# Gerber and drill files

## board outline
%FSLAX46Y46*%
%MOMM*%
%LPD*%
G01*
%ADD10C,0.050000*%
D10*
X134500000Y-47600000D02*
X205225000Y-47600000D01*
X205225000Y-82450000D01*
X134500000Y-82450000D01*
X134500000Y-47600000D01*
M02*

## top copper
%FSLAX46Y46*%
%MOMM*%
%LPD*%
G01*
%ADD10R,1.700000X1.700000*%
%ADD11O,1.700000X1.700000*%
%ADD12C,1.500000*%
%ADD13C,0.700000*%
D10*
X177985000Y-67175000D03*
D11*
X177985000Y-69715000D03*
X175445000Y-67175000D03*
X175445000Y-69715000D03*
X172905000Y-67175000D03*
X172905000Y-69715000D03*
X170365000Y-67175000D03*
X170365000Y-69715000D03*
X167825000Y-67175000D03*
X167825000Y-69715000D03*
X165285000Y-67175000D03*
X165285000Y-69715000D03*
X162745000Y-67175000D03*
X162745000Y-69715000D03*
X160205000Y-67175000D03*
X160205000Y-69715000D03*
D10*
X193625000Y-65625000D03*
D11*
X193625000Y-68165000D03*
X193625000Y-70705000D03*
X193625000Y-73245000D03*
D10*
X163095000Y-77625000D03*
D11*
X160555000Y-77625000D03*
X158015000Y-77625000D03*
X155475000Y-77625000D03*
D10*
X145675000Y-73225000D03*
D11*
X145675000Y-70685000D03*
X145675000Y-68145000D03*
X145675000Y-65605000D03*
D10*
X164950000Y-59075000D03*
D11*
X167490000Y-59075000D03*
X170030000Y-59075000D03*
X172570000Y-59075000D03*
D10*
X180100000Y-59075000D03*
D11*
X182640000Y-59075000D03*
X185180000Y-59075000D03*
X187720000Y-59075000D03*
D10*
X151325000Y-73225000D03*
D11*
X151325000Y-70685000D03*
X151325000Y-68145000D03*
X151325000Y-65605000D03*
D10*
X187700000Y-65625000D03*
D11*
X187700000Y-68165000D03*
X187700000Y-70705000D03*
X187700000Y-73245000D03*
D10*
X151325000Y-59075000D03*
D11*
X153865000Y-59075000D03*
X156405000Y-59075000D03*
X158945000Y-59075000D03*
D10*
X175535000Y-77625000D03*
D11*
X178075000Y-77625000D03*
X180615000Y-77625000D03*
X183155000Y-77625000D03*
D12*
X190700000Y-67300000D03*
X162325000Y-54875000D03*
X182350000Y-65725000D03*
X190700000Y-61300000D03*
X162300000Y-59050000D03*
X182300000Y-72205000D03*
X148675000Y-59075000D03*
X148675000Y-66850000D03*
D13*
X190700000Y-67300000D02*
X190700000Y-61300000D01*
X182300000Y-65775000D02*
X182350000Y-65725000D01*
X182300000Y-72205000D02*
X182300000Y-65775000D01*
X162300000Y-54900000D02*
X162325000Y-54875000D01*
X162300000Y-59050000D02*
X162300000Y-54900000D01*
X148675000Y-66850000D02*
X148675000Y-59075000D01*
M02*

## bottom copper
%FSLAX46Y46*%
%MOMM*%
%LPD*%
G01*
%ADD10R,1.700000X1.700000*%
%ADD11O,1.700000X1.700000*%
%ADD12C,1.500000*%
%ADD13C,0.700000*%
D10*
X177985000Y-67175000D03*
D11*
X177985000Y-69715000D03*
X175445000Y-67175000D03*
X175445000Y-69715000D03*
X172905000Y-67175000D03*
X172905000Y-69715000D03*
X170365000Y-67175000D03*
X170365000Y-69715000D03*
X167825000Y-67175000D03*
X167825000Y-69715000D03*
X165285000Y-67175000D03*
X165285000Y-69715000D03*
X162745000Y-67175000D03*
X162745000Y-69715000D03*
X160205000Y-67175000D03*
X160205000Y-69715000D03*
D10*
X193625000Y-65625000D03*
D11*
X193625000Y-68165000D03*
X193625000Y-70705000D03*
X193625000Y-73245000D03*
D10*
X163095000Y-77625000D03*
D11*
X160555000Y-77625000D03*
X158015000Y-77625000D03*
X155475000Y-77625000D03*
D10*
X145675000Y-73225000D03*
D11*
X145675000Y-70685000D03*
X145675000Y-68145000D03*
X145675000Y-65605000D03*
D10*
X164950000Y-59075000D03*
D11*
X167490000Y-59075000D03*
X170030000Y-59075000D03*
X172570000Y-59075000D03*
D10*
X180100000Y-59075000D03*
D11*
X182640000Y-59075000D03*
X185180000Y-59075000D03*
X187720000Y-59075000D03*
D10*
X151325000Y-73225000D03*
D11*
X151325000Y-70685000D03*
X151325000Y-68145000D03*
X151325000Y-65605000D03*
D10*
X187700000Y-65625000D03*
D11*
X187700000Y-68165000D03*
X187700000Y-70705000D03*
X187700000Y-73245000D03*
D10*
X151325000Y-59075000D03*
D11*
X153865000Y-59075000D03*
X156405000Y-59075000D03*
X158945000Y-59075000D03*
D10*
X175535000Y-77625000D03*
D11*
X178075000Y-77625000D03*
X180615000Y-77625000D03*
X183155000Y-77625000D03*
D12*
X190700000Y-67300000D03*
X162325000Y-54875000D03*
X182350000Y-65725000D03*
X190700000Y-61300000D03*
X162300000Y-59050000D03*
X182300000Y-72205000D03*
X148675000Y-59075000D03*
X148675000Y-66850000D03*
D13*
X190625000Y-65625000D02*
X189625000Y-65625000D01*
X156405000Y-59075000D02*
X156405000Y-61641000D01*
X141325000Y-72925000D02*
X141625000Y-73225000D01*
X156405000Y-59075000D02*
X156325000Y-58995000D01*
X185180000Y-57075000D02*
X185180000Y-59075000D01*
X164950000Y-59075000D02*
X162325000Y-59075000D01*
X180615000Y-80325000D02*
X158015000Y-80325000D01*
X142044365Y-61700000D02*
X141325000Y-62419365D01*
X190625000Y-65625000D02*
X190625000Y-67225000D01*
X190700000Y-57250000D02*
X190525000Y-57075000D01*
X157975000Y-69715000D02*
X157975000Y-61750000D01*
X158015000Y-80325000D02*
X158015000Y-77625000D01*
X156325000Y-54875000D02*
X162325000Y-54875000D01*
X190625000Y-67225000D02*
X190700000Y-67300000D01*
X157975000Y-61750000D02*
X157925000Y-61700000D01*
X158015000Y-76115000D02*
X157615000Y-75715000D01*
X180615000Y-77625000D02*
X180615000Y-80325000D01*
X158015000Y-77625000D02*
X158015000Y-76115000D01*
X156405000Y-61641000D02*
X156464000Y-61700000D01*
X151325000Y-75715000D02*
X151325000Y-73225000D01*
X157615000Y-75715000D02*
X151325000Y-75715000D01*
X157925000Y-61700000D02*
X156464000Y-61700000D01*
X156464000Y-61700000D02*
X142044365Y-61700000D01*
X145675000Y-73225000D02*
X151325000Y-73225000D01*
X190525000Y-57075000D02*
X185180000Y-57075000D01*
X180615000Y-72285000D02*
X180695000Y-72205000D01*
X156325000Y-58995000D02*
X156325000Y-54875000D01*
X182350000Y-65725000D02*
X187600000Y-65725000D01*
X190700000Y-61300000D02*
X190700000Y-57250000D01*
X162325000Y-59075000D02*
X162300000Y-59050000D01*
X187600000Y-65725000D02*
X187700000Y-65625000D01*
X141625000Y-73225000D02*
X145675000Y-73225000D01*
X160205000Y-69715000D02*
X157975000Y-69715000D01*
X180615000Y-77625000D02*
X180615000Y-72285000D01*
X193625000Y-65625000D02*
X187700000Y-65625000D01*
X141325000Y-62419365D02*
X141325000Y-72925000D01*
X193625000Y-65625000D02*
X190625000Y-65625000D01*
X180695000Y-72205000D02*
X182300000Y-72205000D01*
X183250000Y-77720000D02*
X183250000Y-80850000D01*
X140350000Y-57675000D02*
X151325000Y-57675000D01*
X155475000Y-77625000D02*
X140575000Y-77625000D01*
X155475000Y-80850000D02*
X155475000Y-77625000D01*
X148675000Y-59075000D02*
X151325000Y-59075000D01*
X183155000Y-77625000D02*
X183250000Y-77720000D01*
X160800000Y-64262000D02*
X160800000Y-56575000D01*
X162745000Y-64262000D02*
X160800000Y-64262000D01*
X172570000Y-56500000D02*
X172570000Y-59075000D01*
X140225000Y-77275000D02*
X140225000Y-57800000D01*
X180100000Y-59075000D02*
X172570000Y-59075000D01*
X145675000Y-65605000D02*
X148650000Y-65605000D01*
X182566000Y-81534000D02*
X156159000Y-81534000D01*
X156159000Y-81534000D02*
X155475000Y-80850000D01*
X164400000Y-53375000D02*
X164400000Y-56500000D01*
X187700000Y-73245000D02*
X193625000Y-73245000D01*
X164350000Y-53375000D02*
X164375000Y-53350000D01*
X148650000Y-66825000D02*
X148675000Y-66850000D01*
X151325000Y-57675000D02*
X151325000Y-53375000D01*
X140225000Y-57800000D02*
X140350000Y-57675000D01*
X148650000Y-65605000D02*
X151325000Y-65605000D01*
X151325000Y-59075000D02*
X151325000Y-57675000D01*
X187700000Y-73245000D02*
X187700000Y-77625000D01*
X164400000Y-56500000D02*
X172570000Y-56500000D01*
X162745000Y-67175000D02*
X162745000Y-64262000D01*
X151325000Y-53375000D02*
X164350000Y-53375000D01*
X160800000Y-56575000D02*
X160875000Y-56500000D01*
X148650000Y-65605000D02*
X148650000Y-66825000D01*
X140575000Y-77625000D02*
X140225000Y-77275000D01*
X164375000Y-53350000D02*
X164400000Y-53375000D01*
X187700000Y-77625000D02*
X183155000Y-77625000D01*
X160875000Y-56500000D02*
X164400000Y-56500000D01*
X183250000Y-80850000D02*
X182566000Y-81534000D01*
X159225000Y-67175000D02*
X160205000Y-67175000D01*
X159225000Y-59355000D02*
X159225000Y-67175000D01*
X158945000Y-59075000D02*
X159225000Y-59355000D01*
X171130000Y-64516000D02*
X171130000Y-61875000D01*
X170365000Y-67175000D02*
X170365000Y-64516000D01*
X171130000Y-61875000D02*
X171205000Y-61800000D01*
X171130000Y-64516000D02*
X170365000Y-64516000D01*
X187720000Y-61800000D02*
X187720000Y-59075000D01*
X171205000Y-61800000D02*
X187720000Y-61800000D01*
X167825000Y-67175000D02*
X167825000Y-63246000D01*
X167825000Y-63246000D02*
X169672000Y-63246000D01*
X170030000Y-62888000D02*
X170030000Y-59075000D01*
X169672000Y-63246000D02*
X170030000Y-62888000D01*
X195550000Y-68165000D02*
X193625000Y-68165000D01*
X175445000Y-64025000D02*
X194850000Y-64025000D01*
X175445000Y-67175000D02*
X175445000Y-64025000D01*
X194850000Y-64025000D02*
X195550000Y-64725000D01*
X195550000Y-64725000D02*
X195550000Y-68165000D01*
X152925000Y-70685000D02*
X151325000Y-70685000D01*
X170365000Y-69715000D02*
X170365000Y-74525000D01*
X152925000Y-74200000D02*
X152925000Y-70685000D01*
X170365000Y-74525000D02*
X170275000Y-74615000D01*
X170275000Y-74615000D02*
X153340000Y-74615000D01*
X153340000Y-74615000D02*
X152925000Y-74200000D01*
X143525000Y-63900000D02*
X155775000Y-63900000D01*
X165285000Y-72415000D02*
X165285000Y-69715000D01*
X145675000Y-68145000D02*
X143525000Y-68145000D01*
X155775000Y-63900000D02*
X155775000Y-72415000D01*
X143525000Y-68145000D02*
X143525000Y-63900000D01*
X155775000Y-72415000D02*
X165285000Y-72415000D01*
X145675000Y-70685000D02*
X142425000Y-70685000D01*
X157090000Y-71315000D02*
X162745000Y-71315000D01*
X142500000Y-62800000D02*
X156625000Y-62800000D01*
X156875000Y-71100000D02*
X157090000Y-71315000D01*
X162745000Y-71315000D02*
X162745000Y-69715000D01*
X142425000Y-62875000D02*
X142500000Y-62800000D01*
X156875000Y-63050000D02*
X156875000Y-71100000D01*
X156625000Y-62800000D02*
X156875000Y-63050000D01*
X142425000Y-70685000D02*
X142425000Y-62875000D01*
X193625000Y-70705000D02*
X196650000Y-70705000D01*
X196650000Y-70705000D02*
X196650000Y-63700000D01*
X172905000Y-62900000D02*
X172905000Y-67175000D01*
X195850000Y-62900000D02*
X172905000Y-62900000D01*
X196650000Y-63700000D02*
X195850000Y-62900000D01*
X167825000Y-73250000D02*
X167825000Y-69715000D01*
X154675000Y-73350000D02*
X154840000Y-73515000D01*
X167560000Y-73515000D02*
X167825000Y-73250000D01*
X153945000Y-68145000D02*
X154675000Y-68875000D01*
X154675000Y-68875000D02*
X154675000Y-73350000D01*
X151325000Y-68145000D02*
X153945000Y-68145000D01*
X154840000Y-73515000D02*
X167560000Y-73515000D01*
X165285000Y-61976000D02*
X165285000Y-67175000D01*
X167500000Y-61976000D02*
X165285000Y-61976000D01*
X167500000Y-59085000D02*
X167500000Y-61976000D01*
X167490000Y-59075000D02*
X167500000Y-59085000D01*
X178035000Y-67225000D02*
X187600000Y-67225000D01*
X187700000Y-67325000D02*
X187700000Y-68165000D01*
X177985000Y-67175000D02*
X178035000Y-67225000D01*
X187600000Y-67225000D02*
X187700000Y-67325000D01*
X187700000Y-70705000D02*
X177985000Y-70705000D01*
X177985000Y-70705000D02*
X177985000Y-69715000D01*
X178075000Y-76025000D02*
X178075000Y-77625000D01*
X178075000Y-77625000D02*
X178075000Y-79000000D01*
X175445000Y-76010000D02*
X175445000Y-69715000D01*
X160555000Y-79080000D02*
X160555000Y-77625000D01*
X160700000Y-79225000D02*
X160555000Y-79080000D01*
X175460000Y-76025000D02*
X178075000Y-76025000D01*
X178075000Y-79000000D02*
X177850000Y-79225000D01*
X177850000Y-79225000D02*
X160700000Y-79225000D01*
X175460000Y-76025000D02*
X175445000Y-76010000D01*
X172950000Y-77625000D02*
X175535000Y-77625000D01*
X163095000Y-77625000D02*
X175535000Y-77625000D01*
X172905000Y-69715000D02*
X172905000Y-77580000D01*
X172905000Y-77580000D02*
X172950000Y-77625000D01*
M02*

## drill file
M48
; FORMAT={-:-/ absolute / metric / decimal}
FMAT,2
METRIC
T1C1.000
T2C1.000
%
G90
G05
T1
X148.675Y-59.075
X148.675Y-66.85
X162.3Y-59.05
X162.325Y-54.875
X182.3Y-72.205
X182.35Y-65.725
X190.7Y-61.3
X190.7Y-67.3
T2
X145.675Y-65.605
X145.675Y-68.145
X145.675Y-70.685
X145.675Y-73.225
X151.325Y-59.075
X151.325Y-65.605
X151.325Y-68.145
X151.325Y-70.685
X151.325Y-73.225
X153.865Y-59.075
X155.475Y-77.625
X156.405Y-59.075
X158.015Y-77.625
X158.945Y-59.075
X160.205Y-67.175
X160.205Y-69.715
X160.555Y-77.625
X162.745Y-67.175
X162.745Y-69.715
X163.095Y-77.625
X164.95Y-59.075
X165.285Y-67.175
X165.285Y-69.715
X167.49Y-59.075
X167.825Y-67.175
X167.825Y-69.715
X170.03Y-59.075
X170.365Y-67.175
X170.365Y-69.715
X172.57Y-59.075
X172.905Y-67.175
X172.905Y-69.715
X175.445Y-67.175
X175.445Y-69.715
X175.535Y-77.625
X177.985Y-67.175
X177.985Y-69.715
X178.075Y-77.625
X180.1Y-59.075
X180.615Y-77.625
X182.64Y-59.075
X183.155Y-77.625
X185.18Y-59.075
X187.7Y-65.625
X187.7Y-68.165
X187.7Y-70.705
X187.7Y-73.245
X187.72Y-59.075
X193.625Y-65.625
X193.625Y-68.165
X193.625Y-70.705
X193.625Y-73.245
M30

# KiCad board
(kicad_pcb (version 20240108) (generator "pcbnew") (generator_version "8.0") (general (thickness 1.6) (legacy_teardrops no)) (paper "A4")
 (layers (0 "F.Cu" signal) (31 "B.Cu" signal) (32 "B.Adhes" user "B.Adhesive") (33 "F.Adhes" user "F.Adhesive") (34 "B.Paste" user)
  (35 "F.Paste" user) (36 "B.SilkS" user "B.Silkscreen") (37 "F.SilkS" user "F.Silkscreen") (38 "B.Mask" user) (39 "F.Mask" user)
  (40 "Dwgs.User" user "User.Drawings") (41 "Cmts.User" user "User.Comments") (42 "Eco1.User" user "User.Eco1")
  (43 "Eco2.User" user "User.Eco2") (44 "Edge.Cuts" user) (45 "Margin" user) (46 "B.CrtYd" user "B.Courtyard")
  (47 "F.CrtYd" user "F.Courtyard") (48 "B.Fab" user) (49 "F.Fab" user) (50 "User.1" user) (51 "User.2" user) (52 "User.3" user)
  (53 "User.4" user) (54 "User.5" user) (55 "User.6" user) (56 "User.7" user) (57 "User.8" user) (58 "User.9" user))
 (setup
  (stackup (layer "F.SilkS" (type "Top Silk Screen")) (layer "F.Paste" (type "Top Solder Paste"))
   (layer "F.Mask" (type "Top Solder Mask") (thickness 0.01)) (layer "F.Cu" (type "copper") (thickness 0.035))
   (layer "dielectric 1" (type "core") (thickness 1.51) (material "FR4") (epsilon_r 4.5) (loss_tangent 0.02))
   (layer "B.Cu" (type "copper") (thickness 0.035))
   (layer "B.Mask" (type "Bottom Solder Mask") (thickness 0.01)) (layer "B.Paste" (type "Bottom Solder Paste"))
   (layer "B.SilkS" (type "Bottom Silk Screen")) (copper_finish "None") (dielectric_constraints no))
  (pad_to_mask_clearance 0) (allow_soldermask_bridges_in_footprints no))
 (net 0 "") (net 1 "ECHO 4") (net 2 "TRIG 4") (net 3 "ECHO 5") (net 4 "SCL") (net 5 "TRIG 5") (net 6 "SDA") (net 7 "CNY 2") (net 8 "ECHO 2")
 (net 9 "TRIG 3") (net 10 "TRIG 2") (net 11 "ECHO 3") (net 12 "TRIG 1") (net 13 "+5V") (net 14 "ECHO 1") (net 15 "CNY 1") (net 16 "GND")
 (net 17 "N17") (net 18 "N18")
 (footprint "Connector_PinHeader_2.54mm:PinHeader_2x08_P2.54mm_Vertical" (layer "F.Cu") (at 177.985 67.175 -90)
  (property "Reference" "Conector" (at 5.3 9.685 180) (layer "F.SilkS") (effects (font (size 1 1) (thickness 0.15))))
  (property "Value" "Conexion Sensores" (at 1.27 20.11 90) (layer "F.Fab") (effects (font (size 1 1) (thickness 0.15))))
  (pad "1" thru_hole rect (at 0 0 270) (size 1.7 1.7) (drill 1) (layers "*.Cu" "*.Mask") (remove_unused_layers no) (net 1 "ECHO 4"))
  (pad "2" thru_hole oval (at 2.54 0 270) (size 1.7 1.7) (drill 1) (layers "*.Cu" "*.Mask") (remove_unused_layers no) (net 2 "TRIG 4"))
  (pad "3" thru_hole oval (at 0 2.54 270) (size 1.7 1.7) (drill 1) (layers "*.Cu" "*.Mask") (remove_unused_layers no) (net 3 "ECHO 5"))
  (pad "4" thru_hole oval (at 2.54 2.54 270) (size 1.7 1.7) (drill 1) (layers "*.Cu" "*.Mask") (remove_unused_layers no) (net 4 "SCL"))
  (pad "5" thru_hole oval (at 0 5.08 270) (size 1.7 1.7) (drill 1) (layers "*.Cu" "*.Mask") (remove_unused_layers no) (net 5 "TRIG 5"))
  (pad "6" thru_hole oval (at 2.54 5.08 270) (size 1.7 1.7) (drill 1) (layers "*.Cu" "*.Mask") (remove_unused_layers no) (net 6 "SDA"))
  (pad "7" thru_hole oval (at 0 7.62 270) (size 1.7 1.7) (drill 1) (layers "*.Cu" "*.Mask") (remove_unused_layers no) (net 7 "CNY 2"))
  (pad "8" thru_hole oval (at 2.54 7.62 270) (size 1.7 1.7) (drill 1) (layers "*.Cu" "*.Mask") (remove_unused_layers no) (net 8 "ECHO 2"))
  (pad "9" thru_hole oval (at 0 10.16 270) (size 1.7 1.7) (drill 1) (layers "*.Cu" "*.Mask") (remove_unused_layers no) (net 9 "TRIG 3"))
  (pad "10" thru_hole oval (at 2.54 10.16 270) (size 1.7 1.7) (drill 1) (layers "*.Cu" "*.Mask") (remove_unused_layers no) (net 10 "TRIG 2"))
  (pad "11" thru_hole oval (at 0 12.7 270) (size 1.7 1.7) (drill 1) (layers "*.Cu" "*.Mask") (remove_unused_layers no) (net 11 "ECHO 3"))
  (pad "12" thru_hole oval (at 2.54 12.7 270) (size 1.7 1.7) (drill 1) (layers "*.Cu" "*.Mask") (remove_unused_layers no) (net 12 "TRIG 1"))
  (pad "13" thru_hole oval (at 0 15.24 270) (size 1.7 1.7) (drill 1) (layers "*.Cu" "*.Mask") (remove_unused_layers no) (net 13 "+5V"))
  (pad "14" thru_hole oval (at 2.54 15.24 270) (size 1.7 1.7) (drill 1) (layers "*.Cu" "*.Mask") (remove_unused_layers no) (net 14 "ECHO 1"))
  (pad "15" thru_hole oval (at 0 17.78 270) (size 1.7 1.7) (drill 1) (layers "*.Cu" "*.Mask") (remove_unused_layers no) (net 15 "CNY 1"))
  (pad "16" thru_hole oval (at 2.54 17.78 270) (size 1.7 1.7) (drill 1) (layers "*.Cu" "*.Mask") (remove_unused_layers no) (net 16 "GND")))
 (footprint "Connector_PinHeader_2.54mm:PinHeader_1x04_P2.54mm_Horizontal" (layer "F.Cu") (at 193.625 65.625)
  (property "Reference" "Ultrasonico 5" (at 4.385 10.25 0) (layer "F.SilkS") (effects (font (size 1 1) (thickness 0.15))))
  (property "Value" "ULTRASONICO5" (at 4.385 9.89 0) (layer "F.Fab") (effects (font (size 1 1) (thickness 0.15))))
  (pad "1" thru_hole rect (at 0 0) (size 1.7 1.7) (drill 1) (layers "*.Cu" "*.Mask") (remove_unused_layers no) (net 16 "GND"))
  (pad "2" thru_hole oval (at 0 2.54) (size 1.7 1.7) (drill 1) (layers "*.Cu" "*.Mask") (remove_unused_layers no) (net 3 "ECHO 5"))
  (pad "3" thru_hole oval (at 0 5.08) (size 1.7 1.7) (drill 1) (layers "*.Cu" "*.Mask") (remove_unused_layers no) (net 5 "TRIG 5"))
  (pad "4" thru_hole oval (at 0 7.62) (size 1.7 1.7) (drill 1) (layers "*.Cu" "*.Mask") (remove_unused_layers no) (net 13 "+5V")))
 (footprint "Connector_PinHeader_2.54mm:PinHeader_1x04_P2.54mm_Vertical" (layer "F.Cu") (at 163.095 77.625 -90)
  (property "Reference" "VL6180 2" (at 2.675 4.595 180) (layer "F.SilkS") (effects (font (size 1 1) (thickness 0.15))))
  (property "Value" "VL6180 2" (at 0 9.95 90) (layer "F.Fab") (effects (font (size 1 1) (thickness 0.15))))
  (pad "1" thru_hole rect (at 0 0 270) (size 1.7 1.7) (drill 1) (layers "*.Cu" "*.Mask") (remove_unused_layers no) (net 6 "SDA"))
  (pad "2" thru_hole oval (at 0 2.54 270) (size 1.7 1.7) (drill 1) (layers "*.Cu" "*.Mask") (remove_unused_layers no) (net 4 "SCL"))
  (pad "3" thru_hole oval (at 0 5.08 270) (size 1.7 1.7) (drill 1) (layers "*.Cu" "*.Mask") (remove_unused_layers no) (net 16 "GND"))
  (pad "4" thru_hole oval (at 0 7.62 270) (size 1.7 1.7) (drill 1) (layers "*.Cu" "*.Mask") (remove_unused_layers no) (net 13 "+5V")))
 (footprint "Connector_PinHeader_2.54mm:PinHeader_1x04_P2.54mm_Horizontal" (layer "F.Cu") (at 145.675 73.225 180)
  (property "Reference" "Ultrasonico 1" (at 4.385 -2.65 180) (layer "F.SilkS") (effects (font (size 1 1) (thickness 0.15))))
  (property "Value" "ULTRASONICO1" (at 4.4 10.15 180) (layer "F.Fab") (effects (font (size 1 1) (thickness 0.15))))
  (pad "1" thru_hole rect (at 0 0 180) (size 1.7 1.7) (drill 1) (layers "*.Cu" "*.Mask") (remove_unused_layers no) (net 16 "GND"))
  (pad "2" thru_hole oval (at 0 2.54 180) (size 1.7 1.7) (drill 1) (layers "*.Cu" "*.Mask") (remove_unused_layers no) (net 14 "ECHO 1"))
  (pad "3" thru_hole oval (at 0 5.08 180) (size 1.7 1.7) (drill 1) (layers "*.Cu" "*.Mask") (remove_unused_layers no) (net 12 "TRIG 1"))
  (pad "4" thru_hole oval (at 0 7.62 180) (size 1.7 1.7) (drill 1) (layers "*.Cu" "*.Mask") (remove_unused_layers no) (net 13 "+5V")))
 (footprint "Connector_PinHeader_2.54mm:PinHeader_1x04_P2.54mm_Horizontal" (layer "F.Cu") (at 164.95 59.075 90)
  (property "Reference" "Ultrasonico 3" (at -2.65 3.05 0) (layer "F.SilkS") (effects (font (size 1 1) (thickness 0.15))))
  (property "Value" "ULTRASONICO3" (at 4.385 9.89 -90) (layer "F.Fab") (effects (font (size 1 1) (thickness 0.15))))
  (pad "1" thru_hole rect (at 0 0 90) (size 1.7 1.7) (drill 1) (layers "*.Cu" "*.Mask") (remove_unused_layers no) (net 16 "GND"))
  (pad "2" thru_hole oval (at 0 2.54 90) (size 1.7 1.7) (drill 1) (layers "*.Cu" "*.Mask") (remove_unused_layers no) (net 11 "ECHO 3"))
  (pad "3" thru_hole oval (at 0 5.08 90) (size 1.7 1.7) (drill 1) (layers "*.Cu" "*.Mask") (remove_unused_layers no) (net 9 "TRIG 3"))
  (pad "4" thru_hole oval (at 0 7.62 90) (size 1.7 1.7) (drill 1) (layers "*.Cu" "*.Mask") (remove_unused_layers no) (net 13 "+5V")))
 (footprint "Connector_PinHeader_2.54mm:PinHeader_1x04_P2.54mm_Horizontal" (layer "F.Cu") (at 180.1 59.075 90)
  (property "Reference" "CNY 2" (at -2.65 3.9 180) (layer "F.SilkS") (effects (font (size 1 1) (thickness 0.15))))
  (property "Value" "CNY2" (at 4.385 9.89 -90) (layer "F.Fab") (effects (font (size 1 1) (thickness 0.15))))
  (pad "1" thru_hole rect (at 0 0 90) (size 1.7 1.7) (drill 1) (layers "*.Cu" "*.Mask") (remove_unused_layers no) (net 13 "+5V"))
  (pad "2" thru_hole oval (at 0 2.54 90) (size 1.7 1.7) (drill 1) (layers "*.Cu" "*.Mask") (remove_unused_layers no) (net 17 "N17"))
  (pad "3" thru_hole oval (at 0 5.08 90) (size 1.7 1.7) (drill 1) (layers "*.Cu" "*.Mask") (remove_unused_layers no) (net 16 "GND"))
  (pad "4" thru_hole oval (at 0 7.62 90) (size 1.7 1.7) (drill 1) (layers "*.Cu" "*.Mask") (remove_unused_layers no) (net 7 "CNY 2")))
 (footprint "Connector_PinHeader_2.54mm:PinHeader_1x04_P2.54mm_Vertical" (layer "F.Cu") (at 151.325 73.225 180)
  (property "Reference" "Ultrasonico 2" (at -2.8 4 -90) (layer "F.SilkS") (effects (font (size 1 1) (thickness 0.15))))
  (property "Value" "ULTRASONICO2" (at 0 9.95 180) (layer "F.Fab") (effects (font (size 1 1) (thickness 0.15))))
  (pad "1" thru_hole rect (at 0 0 180) (size 1.7 1.7) (drill 1) (layers "*.Cu" "*.Mask") (remove_unused_layers no) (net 16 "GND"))
  (pad "2" thru_hole oval (at 0 2.54 180) (size 1.7 1.7) (drill 1) (layers "*.Cu" "*.Mask") (remove_unused_layers no) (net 8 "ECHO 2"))
  (pad "3" thru_hole oval (at 0 5.08 180) (size 1.7 1.7) (drill 1) (layers "*.Cu" "*.Mask") (remove_unused_layers no) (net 10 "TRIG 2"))
  (pad "4" thru_hole oval (at 0 7.62 180) (size 1.7 1.7) (drill 1) (layers "*.Cu" "*.Mask") (remove_unused_layers no) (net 13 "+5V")))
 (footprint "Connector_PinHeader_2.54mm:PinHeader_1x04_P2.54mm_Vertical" (layer "F.Cu") (at 187.7 65.625)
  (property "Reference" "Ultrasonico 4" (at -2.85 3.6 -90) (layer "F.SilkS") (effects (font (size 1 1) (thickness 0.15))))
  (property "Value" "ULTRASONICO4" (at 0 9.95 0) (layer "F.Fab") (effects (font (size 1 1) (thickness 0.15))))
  (pad "1" thru_hole rect (at 0 0) (size 1.7 1.7) (drill 1) (layers "*.Cu" "*.Mask") (remove_unused_layers no) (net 16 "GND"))
  (pad "2" thru_hole oval (at 0 2.54) (size 1.7 1.7) (drill 1) (layers "*.Cu" "*.Mask") (remove_unused_layers no) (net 1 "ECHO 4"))
  (pad "3" thru_hole oval (at 0 5.08) (size 1.7 1.7) (drill 1) (layers "*.Cu" "*.Mask") (remove_unused_layers no) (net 2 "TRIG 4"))
  (pad "4" thru_hole oval (at 0 7.62) (size 1.7 1.7) (drill 1) (layers "*.Cu" "*.Mask") (remove_unused_layers no) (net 13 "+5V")))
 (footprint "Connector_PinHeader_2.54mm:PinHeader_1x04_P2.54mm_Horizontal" (layer "F.Cu") (at 151.325 59.075 90)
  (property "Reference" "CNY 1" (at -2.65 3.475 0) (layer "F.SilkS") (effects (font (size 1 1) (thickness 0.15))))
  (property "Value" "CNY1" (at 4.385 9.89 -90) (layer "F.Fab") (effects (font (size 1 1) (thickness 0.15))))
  (pad "1" thru_hole rect (at 0 0 90) (size 1.7 1.7) (drill 1) (layers "*.Cu" "*.Mask") (remove_unused_layers no) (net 13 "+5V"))
  (pad "2" thru_hole oval (at 0 2.54 90) (size 1.7 1.7) (drill 1) (layers "*.Cu" "*.Mask") (remove_unused_layers no) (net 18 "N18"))
  (pad "3" thru_hole oval (at 0 5.08 90) (size 1.7 1.7) (drill 1) (layers "*.Cu" "*.Mask") (remove_unused_layers no) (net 16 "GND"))
  (pad "4" thru_hole oval (at 0 7.62 90) (size 1.7 1.7) (drill 1) (layers "*.Cu" "*.Mask") (remove_unused_layers no) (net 15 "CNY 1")))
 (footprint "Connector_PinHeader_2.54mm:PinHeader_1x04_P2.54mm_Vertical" (layer "F.Cu") (at 175.535 77.625 90)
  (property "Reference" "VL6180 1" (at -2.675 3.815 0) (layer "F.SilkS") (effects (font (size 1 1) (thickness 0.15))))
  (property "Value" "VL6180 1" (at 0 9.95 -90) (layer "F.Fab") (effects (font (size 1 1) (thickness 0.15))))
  (pad "1" thru_hole rect (at 0 0 90) (size 1.7 1.7) (drill 1) (layers "*.Cu" "*.Mask") (remove_unused_layers no) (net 6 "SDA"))
  (pad "2" thru_hole oval (at 0 2.54 90) (size 1.7 1.7) (drill 1) (layers "*.Cu" "*.Mask") (remove_unused_layers no) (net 4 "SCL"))
  (pad "3" thru_hole oval (at 0 5.08 90) (size 1.7 1.7) (drill 1) (layers "*.Cu" "*.Mask") (remove_unused_layers no) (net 16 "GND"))
  (pad "4" thru_hole oval (at 0 7.62 90) (size 1.7 1.7) (drill 1) (layers "*.Cu" "*.Mask") (remove_unused_layers no) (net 13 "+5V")))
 (gr_rect (start 134.5 47.6) (end 205.225 82.45) (stroke (width 0.05) (type default)) (fill none) (layer "Edge.Cuts"))
 (segment (start 190.7 67.3) (end 190.7 61.3) (width 0.7) (layer "F.Cu") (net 16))
 (segment (start 182.3 65.775) (end 182.35 65.725) (width 0.7) (layer "F.Cu") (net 16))
 (segment (start 182.3 72.205) (end 182.3 65.775) (width 0.7) (layer "F.Cu") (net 16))
 (segment (start 162.3 54.9) (end 162.325 54.875) (width 0.7) (layer "F.Cu") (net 16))
 (segment (start 162.3 59.05) (end 162.3 54.9) (width 0.7) (layer "F.Cu") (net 16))
 (via (at 190.7 67.3) (size 1.5) (drill 1) (layers "F.Cu" "B.Cu") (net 16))
 (via (at 162.325 54.875) (size 1.5) (drill 1) (layers "F.Cu" "B.Cu") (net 16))
 (via (at 182.35 65.725) (size 1.5) (drill 1) (layers "F.Cu" "B.Cu") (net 16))
 (via (at 190.7 61.3) (size 1.5) (drill 1) (layers "F.Cu" "B.Cu") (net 16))
 (via (at 162.3 59.05) (size 1.5) (drill 1) (layers "F.Cu" "B.Cu") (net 16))
 (via (at 182.3 72.205) (size 1.5) (drill 1) (layers "F.Cu" "B.Cu") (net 16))
 (segment (start 190.625 65.625) (end 189.625 65.625) (width 0.7) (layer "B.Cu") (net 16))
 (segment (start 156.405 59.075) (end 156.405 61.641) (width 0.7) (layer "B.Cu") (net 16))
 (segment (start 141.325 72.925) (end 141.625 73.225) (width 0.7) (layer "B.Cu") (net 16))
 (segment (start 156.405 59.075) (end 156.325 58.995) (width 0.7) (layer "B.Cu") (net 16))
 (segment (start 185.18 57.075) (end 185.18 59.075) (width 0.7) (layer "B.Cu") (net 16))
 (segment (start 164.95 59.075) (end 162.325 59.075) (width 0.7) (layer "B.Cu") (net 16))
 (segment (start 180.615 80.325) (end 158.015 80.325) (width 0.7) (layer "B.Cu") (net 16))
 (segment (start 142.044365 61.7) (end 141.325 62.419365) (width 0.7) (layer "B.Cu") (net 16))
 (segment (start 190.625 65.625) (end 190.625 67.225) (width 0.7) (layer "B.Cu") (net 16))
 (segment (start 190.7 57.25) (end 190.525 57.075) (width 0.7) (layer "B.Cu") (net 16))
 (segment (start 157.975 69.715) (end 157.975 61.75) (width 0.7) (layer "B.Cu") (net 16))
 (segment (start 158.015 80.325) (end 158.015 77.625) (width 0.7) (layer "B.Cu") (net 16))
 (segment (start 156.325 54.875) (end 162.325 54.875) (width 0.7) (layer "B.Cu") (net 16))
 (segment (start 190.625 67.225) (end 190.7 67.3) (width 0.7) (layer "B.Cu") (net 16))
 (segment (start 157.975 61.75) (end 157.925 61.7) (width 0.7) (layer "B.Cu") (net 16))
 (segment (start 158.015 76.115) (end 157.615 75.715) (width 0.7) (layer "B.Cu") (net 16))
 (segment (start 180.615 77.625) (end 180.615 80.325) (width 0.7) (layer "B.Cu") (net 16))
 (segment (start 158.015 77.625) (end 158.015 76.115) (width 0.7) (layer "B.Cu") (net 16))
 (segment (start 156.405 61.641) (end 156.464 61.7) (width 0.7) (layer "B.Cu") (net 16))
 (segment (start 151.325 75.715) (end 151.325 73.225) (width 0.7) (layer "B.Cu") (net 16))
 (segment (start 157.615 75.715) (end 151.325 75.715) (width 0.7) (layer "B.Cu") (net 16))
 (segment (start 157.925 61.7) (end 156.464 61.7) (width 0.7) (layer "B.Cu") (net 16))
 (segment (start 156.464 61.7) (end 142.044365 61.7) (width 0.7) (layer "B.Cu") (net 16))
 (segment (start 145.675 73.225) (end 151.325 73.225) (width 0.7) (layer "B.Cu") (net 16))
 (segment (start 190.525 57.075) (end 185.18 57.075) (width 0.7) (layer "B.Cu") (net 16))
 (segment (start 180.615 72.285) (end 180.695 72.205) (width 0.7) (layer "B.Cu") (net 16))
 (segment (start 156.325 58.995) (end 156.325 54.875) (width 0.7) (layer "B.Cu") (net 16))
 (segment (start 182.35 65.725) (end 187.6 65.725) (width 0.7) (layer "B.Cu") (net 16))
 (segment (start 190.7 61.3) (end 190.7 57.25) (width 0.7) (layer "B.Cu") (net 16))
 (segment (start 162.325 59.075) (end 162.3 59.05) (width 0.7) (layer "B.Cu") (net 16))
 (segment (start 187.6 65.725) (end 187.7 65.625) (width 0.7) (layer "B.Cu") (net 16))
 (segment (start 141.625 73.225) (end 145.675 73.225) (width 0.7) (layer "B.Cu") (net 16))
 (segment (start 160.205 69.715) (end 157.975 69.715) (width 0.7) (layer "B.Cu") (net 16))
 (segment (start 180.615 77.625) (end 180.615 72.285) (width 0.7) (layer "B.Cu") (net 16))
 (segment (start 193.625 65.625) (end 187.7 65.625) (width 0.7) (layer "B.Cu") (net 16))
 (segment (start 141.325 62.419365) (end 141.325 72.925) (width 0.7) (layer "B.Cu") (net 16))
 (segment (start 193.625 65.625) (end 190.625 65.625) (width 0.7) (layer "B.Cu") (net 16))
 (segment (start 180.695 72.205) (end 182.3 72.205) (width 0.7) (layer "B.Cu") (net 16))
 (segment (start 148.675 66.85) (end 148.675 59.075) (width 0.7) (layer "F.Cu") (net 13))
 (via (at 148.675 59.075) (size 1.5) (drill 1) (layers "F.Cu" "B.Cu") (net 13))
 (via (at 148.675 66.85) (size 1.5) (drill 1) (layers "F.Cu" "B.Cu") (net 13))
 (segment (start 183.25 77.72) (end 183.25 80.85) (width 0.7) (layer "B.Cu") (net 13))
 (segment (start 140.35 57.675) (end 151.325 57.675) (width 0.7) (layer "B.Cu") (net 13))
 (segment (start 155.475 77.625) (end 140.575 77.625) (width 0.7) (layer "B.Cu") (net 13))
 (segment (start 155.475 80.85) (end 155.475 77.625) (width 0.7) (layer "B.Cu") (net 13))
 (segment (start 148.675 59.075) (end 151.325 59.075) (width 0.7) (layer "B.Cu") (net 13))
 (segment (start 183.155 77.625) (end 183.25 77.72) (width 0.7) (layer "B.Cu") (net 13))
 (segment (start 160.8 64.262) (end 160.8 56.575) (width 0.7) (layer "B.Cu") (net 13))
 (segment (start 162.745 64.262) (end 160.8 64.262) (width 0.7) (layer "B.Cu") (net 13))
 (segment (start 172.57 56.5) (end 172.57 59.075) (width 0.7) (layer "B.Cu") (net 13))
 (segment (start 140.225 77.275) (end 140.225 57.8) (width 0.7) (layer "B.Cu") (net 13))
 (segment (start 180.1 59.075) (end 172.57 59.075) (width 0.7) (layer "B.Cu") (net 13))
 (segment (start 145.675 65.605) (end 148.65 65.605) (width 0.7) (layer "B.Cu") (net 13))
 (segment (start 182.566 81.534) (end 156.159 81.534) (width 0.7) (layer "B.Cu") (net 13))
 (segment (start 156.159 81.534) (end 155.475 80.85) (width 0.7) (layer "B.Cu") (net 13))
 (segment (start 164.4 53.375) (end 164.4 56.5) (width 0.7) (layer "B.Cu") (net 13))
 (segment (start 187.7 73.245) (end 193.625 73.245) (width 0.7) (layer "B.Cu") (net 13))
 (segment (start 164.35 53.375) (end 164.375 53.35) (width 0.7) (layer "B.Cu") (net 13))
 (segment (start 148.65 66.825) (end 148.675 66.85) (width 0.7) (layer "B.Cu") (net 13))
 (segment (start 151.325 57.675) (end 151.325 53.375) (width 0.7) (layer "B.Cu") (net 13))
 (segment (start 140.225 57.8) (end 140.35 57.675) (width 0.7) (layer "B.Cu") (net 13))
 (segment (start 148.65 65.605) (end 151.325 65.605) (width 0.7) (layer "B.Cu") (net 13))
 (segment (start 151.325 59.075) (end 151.325 57.675) (width 0.7) (layer "B.Cu") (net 13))
 (segment (start 187.7 73.245) (end 187.7 77.625) (width 0.7) (layer "B.Cu") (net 13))
 (segment (start 164.4 56.5) (end 172.57 56.5) (width 0.7) (layer "B.Cu") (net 13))
 (segment (start 162.745 67.175) (end 162.745 64.262) (width 0.7) (layer "B.Cu") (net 13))
 (segment (start 151.325 53.375) (end 164.35 53.375) (width 0.7) (layer "B.Cu") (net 13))
 (segment (start 160.8 56.575) (end 160.875 56.5) (width 0.7) (layer "B.Cu") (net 13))
 (segment (start 148.65 65.605) (end 148.65 66.825) (width 0.7) (layer "B.Cu") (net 13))
 (segment (start 140.575 77.625) (end 140.225 77.275) (width 0.7) (layer "B.Cu") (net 13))
 (segment (start 164.375 53.35) (end 164.4 53.375) (width 0.7) (layer "B.Cu") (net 13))
 (segment (start 187.7 77.625) (end 183.155 77.625) (width 0.7) (layer "B.Cu") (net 13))
 (segment (start 160.875 56.5) (end 164.4 56.5) (width 0.7) (layer "B.Cu") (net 13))
 (segment (start 183.25 80.85) (end 182.566 81.534) (width 0.7) (layer "B.Cu") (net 13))
 (segment (start 159.225 67.175) (end 160.205 67.175) (width 0.7) (layer "B.Cu") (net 15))
 (segment (start 159.225 59.355) (end 159.225 67.175) (width 0.7) (layer "B.Cu") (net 15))
 (segment (start 158.945 59.075) (end 159.225 59.355) (width 0.7) (layer "B.Cu") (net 15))
 (segment (start 171.13 64.516) (end 171.13 61.875) (width 0.7) (layer "B.Cu") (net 7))
 (segment (start 170.365 67.175) (end 170.365 64.516) (width 0.7) (layer "B.Cu") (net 7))
 (segment (start 171.13 61.875) (end 171.205 61.8) (width 0.7) (layer "B.Cu") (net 7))
 (segment (start 171.13 64.516) (end 170.365 64.516) (width 0.7) (layer "B.Cu") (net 7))
 (segment (start 187.72 61.8) (end 187.72 59.075) (width 0.7) (layer "B.Cu") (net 7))
 (segment (start 171.205 61.8) (end 187.72 61.8) (width 0.7) (layer "B.Cu") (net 7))
 (segment (start 167.825 67.175) (end 167.825 63.246) (width 0.7) (layer "B.Cu") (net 9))
 (segment (start 167.825 63.246) (end 169.672 63.246) (width 0.7) (layer "B.Cu") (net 9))
 (segment (start 170.03 62.888) (end 170.03 59.075) (width 0.7) (layer "B.Cu") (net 9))
 (segment (start 169.672 63.246) (end 170.03 62.888) (width 0.7) (layer "B.Cu") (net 9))
 (segment (start 195.55 68.165) (end 193.625 68.165) (width 0.7) (layer "B.Cu") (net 3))
 (segment (start 175.445 64.025) (end 194.85 64.025) (width 0.7) (layer "B.Cu") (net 3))
 (segment (start 175.445 67.175) (end 175.445 64.025) (width 0.7) (layer "B.Cu") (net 3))
 (segment (start 194.85 64.025) (end 195.55 64.725) (width 0.7) (layer "B.Cu") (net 3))
 (segment (start 195.55 64.725) (end 195.55 68.165) (width 0.7) (layer "B.Cu") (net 3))
 (segment (start 152.925 70.685) (end 151.325 70.685) (width 0.7) (layer "B.Cu") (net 8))
 (segment (start 170.365 69.715) (end 170.365 74.525) (width 0.7) (layer "B.Cu") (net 8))
 (segment (start 152.925 74.2) (end 152.925 70.685) (width 0.7) (layer "B.Cu") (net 8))
 (segment (start 170.365 74.525) (end 170.275 74.615) (width 0.7) (layer "B.Cu") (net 8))
 (segment (start 170.275 74.615) (end 153.34 74.615) (width 0.7) (layer "B.Cu") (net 8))
 (segment (start 153.34 74.615) (end 152.925 74.2) (width 0.7) (layer "B.Cu") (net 8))
 (segment (start 143.525 63.9) (end 155.775 63.9) (width 0.7) (layer "B.Cu") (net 12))
 (segment (start 165.285 72.415) (end 165.285 69.715) (width 0.7) (layer "B.Cu") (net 12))
 (segment (start 145.675 68.145) (end 143.525 68.145) (width 0.7) (layer "B.Cu") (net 12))
 (segment (start 155.775 63.9) (end 155.775 72.415) (width 0.7) (layer "B.Cu") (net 12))
 (segment (start 143.525 68.145) (end 143.525 63.9) (width 0.7) (layer "B.Cu") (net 12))
 (segment (start 155.775 72.415) (end 165.285 72.415) (width 0.7) (layer "B.Cu") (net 12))
 (segment (start 145.675 70.685) (end 142.425 70.685) (width 0.7) (layer "B.Cu") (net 14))
 (segment (start 157.09 71.315) (end 162.745 71.315) (width 0.7) (layer "B.Cu") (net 14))
 (segment (start 142.5 62.8) (end 156.625 62.8) (width 0.7) (layer "B.Cu") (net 14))
 (segment (start 156.875 71.1) (end 157.09 71.315) (width 0.7) (layer "B.Cu") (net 14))
 (segment (start 162.745 71.315) (end 162.745 69.715) (width 0.7) (layer "B.Cu") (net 14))
 (segment (start 142.425 62.875) (end 142.5 62.8) (width 0.7) (layer "B.Cu") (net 14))
 (segment (start 156.875 63.05) (end 156.875 71.1) (width 0.7) (layer "B.Cu") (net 14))
 (segment (start 156.625 62.8) (end 156.875 63.05) (width 0.7) (layer "B.Cu") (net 14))
 (segment (start 142.425 70.685) (end 142.425 62.875) (width 0.7) (layer "B.Cu") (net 14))
 (segment (start 193.625 70.705) (end 196.65 70.705) (width 0.7) (layer "B.Cu") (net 5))
 (segment (start 196.65 70.705) (end 196.65 63.7) (width 0.7) (layer "B.Cu") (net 5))
 (segment (start 172.905 62.9) (end 172.905 67.175) (width 0.7) (layer "B.Cu") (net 5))
 (segment (start 195.85 62.9) (end 172.905 62.9) (width 0.7) (layer "B.Cu") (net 5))
 (segment (start 196.65 63.7) (end 195.85 62.9) (width 0.7) (layer "B.Cu") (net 5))
 (segment (start 167.825 73.25) (end 167.825 69.715) (width 0.7) (layer "B.Cu") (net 10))
 (segment (start 154.675 73.35) (end 154.84 73.515) (width 0.7) (layer "B.Cu") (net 10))
 (segment (start 167.56 73.515) (end 167.825 73.25) (width 0.7) (layer "B.Cu") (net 10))
 (segment (start 153.945 68.145) (end 154.675 68.875) (width 0.7) (layer "B.Cu") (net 10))
 (segment (start 154.675 68.875) (end 154.675 73.35) (width 0.7) (layer "B.Cu") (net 10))
 (segment (start 151.325 68.145) (end 153.945 68.145) (width 0.7) (layer "B.Cu") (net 10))
 (segment (start 154.84 73.515) (end 167.56 73.515) (width 0.7) (layer "B.Cu") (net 10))
 (segment (start 165.285 61.976) (end 165.285 67.175) (width 0.7) (layer "B.Cu") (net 11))
 (segment (start 167.5 61.976) (end 165.285 61.976) (width 0.7) (layer "B.Cu") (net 11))
 (segment (start 167.5 59.085) (end 167.5 61.976) (width 0.7) (layer "B.Cu") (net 11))
 (segment (start 167.49 59.075) (end 167.5 59.085) (width 0.7) (layer "B.Cu") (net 11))
 (segment (start 178.035 67.225) (end 187.6 67.225) (width 0.7) (layer "B.Cu") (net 1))
 (segment (start 187.7 67.325) (end 187.7 68.165) (width 0.7) (layer "B.Cu") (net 1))
 (segment (start 177.985 67.175) (end 178.035 67.225) (width 0.7) (layer "B.Cu") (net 1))
 (segment (start 187.6 67.225) (end 187.7 67.325) (width 0.7) (layer "B.Cu") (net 1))
 (segment (start 187.7 70.705) (end 177.985 70.705) (width 0.7) (layer "B.Cu") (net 2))
 (segment (start 177.985 70.705) (end 177.985 69.715) (width 0.7) (layer "B.Cu") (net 2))
 (segment (start 178.075 76.025) (end 178.075 77.625) (width 0.7) (layer "B.Cu") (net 4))
 (segment (start 178.075 77.625) (end 178.075 79) (width 0.7) (layer "B.Cu") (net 4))
 (segment (start 175.445 76.01) (end 175.445 69.715) (width 0.7) (layer "B.Cu") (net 4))
 (segment (start 160.555 79.08) (end 160.555 77.625) (width 0.7) (layer "B.Cu") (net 4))
 (segment (start 160.7 79.225) (end 160.555 79.08) (width 0.7) (layer "B.Cu") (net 4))
 (segment (start 175.46 76.025) (end 178.075 76.025) (width 0.7) (layer "B.Cu") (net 4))
 (segment (start 178.075 79) (end 177.85 79.225) (width 0.7) (layer "B.Cu") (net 4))
 (segment (start 177.85 79.225) (end 160.7 79.225) (width 0.7) (layer "B.Cu") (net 4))
 (segment (start 175.46 76.025) (end 175.445 76.01) (width 0.7) (layer "B.Cu") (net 4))
 (segment (start 172.95 77.625) (end 175.535 77.625) (width 0.7) (layer "B.Cu") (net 6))
 (segment (start 163.095 77.625) (end 175.535 77.625) (width 0.7) (layer "B.Cu") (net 6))
 (segment (start 172.905 69.715) (end 172.905 77.58) (width 0.7) (layer "B.Cu") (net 6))
 (segment (start 172.905 77.58) (end 172.95 77.625) (width 0.7) (layer "B.Cu") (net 6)))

